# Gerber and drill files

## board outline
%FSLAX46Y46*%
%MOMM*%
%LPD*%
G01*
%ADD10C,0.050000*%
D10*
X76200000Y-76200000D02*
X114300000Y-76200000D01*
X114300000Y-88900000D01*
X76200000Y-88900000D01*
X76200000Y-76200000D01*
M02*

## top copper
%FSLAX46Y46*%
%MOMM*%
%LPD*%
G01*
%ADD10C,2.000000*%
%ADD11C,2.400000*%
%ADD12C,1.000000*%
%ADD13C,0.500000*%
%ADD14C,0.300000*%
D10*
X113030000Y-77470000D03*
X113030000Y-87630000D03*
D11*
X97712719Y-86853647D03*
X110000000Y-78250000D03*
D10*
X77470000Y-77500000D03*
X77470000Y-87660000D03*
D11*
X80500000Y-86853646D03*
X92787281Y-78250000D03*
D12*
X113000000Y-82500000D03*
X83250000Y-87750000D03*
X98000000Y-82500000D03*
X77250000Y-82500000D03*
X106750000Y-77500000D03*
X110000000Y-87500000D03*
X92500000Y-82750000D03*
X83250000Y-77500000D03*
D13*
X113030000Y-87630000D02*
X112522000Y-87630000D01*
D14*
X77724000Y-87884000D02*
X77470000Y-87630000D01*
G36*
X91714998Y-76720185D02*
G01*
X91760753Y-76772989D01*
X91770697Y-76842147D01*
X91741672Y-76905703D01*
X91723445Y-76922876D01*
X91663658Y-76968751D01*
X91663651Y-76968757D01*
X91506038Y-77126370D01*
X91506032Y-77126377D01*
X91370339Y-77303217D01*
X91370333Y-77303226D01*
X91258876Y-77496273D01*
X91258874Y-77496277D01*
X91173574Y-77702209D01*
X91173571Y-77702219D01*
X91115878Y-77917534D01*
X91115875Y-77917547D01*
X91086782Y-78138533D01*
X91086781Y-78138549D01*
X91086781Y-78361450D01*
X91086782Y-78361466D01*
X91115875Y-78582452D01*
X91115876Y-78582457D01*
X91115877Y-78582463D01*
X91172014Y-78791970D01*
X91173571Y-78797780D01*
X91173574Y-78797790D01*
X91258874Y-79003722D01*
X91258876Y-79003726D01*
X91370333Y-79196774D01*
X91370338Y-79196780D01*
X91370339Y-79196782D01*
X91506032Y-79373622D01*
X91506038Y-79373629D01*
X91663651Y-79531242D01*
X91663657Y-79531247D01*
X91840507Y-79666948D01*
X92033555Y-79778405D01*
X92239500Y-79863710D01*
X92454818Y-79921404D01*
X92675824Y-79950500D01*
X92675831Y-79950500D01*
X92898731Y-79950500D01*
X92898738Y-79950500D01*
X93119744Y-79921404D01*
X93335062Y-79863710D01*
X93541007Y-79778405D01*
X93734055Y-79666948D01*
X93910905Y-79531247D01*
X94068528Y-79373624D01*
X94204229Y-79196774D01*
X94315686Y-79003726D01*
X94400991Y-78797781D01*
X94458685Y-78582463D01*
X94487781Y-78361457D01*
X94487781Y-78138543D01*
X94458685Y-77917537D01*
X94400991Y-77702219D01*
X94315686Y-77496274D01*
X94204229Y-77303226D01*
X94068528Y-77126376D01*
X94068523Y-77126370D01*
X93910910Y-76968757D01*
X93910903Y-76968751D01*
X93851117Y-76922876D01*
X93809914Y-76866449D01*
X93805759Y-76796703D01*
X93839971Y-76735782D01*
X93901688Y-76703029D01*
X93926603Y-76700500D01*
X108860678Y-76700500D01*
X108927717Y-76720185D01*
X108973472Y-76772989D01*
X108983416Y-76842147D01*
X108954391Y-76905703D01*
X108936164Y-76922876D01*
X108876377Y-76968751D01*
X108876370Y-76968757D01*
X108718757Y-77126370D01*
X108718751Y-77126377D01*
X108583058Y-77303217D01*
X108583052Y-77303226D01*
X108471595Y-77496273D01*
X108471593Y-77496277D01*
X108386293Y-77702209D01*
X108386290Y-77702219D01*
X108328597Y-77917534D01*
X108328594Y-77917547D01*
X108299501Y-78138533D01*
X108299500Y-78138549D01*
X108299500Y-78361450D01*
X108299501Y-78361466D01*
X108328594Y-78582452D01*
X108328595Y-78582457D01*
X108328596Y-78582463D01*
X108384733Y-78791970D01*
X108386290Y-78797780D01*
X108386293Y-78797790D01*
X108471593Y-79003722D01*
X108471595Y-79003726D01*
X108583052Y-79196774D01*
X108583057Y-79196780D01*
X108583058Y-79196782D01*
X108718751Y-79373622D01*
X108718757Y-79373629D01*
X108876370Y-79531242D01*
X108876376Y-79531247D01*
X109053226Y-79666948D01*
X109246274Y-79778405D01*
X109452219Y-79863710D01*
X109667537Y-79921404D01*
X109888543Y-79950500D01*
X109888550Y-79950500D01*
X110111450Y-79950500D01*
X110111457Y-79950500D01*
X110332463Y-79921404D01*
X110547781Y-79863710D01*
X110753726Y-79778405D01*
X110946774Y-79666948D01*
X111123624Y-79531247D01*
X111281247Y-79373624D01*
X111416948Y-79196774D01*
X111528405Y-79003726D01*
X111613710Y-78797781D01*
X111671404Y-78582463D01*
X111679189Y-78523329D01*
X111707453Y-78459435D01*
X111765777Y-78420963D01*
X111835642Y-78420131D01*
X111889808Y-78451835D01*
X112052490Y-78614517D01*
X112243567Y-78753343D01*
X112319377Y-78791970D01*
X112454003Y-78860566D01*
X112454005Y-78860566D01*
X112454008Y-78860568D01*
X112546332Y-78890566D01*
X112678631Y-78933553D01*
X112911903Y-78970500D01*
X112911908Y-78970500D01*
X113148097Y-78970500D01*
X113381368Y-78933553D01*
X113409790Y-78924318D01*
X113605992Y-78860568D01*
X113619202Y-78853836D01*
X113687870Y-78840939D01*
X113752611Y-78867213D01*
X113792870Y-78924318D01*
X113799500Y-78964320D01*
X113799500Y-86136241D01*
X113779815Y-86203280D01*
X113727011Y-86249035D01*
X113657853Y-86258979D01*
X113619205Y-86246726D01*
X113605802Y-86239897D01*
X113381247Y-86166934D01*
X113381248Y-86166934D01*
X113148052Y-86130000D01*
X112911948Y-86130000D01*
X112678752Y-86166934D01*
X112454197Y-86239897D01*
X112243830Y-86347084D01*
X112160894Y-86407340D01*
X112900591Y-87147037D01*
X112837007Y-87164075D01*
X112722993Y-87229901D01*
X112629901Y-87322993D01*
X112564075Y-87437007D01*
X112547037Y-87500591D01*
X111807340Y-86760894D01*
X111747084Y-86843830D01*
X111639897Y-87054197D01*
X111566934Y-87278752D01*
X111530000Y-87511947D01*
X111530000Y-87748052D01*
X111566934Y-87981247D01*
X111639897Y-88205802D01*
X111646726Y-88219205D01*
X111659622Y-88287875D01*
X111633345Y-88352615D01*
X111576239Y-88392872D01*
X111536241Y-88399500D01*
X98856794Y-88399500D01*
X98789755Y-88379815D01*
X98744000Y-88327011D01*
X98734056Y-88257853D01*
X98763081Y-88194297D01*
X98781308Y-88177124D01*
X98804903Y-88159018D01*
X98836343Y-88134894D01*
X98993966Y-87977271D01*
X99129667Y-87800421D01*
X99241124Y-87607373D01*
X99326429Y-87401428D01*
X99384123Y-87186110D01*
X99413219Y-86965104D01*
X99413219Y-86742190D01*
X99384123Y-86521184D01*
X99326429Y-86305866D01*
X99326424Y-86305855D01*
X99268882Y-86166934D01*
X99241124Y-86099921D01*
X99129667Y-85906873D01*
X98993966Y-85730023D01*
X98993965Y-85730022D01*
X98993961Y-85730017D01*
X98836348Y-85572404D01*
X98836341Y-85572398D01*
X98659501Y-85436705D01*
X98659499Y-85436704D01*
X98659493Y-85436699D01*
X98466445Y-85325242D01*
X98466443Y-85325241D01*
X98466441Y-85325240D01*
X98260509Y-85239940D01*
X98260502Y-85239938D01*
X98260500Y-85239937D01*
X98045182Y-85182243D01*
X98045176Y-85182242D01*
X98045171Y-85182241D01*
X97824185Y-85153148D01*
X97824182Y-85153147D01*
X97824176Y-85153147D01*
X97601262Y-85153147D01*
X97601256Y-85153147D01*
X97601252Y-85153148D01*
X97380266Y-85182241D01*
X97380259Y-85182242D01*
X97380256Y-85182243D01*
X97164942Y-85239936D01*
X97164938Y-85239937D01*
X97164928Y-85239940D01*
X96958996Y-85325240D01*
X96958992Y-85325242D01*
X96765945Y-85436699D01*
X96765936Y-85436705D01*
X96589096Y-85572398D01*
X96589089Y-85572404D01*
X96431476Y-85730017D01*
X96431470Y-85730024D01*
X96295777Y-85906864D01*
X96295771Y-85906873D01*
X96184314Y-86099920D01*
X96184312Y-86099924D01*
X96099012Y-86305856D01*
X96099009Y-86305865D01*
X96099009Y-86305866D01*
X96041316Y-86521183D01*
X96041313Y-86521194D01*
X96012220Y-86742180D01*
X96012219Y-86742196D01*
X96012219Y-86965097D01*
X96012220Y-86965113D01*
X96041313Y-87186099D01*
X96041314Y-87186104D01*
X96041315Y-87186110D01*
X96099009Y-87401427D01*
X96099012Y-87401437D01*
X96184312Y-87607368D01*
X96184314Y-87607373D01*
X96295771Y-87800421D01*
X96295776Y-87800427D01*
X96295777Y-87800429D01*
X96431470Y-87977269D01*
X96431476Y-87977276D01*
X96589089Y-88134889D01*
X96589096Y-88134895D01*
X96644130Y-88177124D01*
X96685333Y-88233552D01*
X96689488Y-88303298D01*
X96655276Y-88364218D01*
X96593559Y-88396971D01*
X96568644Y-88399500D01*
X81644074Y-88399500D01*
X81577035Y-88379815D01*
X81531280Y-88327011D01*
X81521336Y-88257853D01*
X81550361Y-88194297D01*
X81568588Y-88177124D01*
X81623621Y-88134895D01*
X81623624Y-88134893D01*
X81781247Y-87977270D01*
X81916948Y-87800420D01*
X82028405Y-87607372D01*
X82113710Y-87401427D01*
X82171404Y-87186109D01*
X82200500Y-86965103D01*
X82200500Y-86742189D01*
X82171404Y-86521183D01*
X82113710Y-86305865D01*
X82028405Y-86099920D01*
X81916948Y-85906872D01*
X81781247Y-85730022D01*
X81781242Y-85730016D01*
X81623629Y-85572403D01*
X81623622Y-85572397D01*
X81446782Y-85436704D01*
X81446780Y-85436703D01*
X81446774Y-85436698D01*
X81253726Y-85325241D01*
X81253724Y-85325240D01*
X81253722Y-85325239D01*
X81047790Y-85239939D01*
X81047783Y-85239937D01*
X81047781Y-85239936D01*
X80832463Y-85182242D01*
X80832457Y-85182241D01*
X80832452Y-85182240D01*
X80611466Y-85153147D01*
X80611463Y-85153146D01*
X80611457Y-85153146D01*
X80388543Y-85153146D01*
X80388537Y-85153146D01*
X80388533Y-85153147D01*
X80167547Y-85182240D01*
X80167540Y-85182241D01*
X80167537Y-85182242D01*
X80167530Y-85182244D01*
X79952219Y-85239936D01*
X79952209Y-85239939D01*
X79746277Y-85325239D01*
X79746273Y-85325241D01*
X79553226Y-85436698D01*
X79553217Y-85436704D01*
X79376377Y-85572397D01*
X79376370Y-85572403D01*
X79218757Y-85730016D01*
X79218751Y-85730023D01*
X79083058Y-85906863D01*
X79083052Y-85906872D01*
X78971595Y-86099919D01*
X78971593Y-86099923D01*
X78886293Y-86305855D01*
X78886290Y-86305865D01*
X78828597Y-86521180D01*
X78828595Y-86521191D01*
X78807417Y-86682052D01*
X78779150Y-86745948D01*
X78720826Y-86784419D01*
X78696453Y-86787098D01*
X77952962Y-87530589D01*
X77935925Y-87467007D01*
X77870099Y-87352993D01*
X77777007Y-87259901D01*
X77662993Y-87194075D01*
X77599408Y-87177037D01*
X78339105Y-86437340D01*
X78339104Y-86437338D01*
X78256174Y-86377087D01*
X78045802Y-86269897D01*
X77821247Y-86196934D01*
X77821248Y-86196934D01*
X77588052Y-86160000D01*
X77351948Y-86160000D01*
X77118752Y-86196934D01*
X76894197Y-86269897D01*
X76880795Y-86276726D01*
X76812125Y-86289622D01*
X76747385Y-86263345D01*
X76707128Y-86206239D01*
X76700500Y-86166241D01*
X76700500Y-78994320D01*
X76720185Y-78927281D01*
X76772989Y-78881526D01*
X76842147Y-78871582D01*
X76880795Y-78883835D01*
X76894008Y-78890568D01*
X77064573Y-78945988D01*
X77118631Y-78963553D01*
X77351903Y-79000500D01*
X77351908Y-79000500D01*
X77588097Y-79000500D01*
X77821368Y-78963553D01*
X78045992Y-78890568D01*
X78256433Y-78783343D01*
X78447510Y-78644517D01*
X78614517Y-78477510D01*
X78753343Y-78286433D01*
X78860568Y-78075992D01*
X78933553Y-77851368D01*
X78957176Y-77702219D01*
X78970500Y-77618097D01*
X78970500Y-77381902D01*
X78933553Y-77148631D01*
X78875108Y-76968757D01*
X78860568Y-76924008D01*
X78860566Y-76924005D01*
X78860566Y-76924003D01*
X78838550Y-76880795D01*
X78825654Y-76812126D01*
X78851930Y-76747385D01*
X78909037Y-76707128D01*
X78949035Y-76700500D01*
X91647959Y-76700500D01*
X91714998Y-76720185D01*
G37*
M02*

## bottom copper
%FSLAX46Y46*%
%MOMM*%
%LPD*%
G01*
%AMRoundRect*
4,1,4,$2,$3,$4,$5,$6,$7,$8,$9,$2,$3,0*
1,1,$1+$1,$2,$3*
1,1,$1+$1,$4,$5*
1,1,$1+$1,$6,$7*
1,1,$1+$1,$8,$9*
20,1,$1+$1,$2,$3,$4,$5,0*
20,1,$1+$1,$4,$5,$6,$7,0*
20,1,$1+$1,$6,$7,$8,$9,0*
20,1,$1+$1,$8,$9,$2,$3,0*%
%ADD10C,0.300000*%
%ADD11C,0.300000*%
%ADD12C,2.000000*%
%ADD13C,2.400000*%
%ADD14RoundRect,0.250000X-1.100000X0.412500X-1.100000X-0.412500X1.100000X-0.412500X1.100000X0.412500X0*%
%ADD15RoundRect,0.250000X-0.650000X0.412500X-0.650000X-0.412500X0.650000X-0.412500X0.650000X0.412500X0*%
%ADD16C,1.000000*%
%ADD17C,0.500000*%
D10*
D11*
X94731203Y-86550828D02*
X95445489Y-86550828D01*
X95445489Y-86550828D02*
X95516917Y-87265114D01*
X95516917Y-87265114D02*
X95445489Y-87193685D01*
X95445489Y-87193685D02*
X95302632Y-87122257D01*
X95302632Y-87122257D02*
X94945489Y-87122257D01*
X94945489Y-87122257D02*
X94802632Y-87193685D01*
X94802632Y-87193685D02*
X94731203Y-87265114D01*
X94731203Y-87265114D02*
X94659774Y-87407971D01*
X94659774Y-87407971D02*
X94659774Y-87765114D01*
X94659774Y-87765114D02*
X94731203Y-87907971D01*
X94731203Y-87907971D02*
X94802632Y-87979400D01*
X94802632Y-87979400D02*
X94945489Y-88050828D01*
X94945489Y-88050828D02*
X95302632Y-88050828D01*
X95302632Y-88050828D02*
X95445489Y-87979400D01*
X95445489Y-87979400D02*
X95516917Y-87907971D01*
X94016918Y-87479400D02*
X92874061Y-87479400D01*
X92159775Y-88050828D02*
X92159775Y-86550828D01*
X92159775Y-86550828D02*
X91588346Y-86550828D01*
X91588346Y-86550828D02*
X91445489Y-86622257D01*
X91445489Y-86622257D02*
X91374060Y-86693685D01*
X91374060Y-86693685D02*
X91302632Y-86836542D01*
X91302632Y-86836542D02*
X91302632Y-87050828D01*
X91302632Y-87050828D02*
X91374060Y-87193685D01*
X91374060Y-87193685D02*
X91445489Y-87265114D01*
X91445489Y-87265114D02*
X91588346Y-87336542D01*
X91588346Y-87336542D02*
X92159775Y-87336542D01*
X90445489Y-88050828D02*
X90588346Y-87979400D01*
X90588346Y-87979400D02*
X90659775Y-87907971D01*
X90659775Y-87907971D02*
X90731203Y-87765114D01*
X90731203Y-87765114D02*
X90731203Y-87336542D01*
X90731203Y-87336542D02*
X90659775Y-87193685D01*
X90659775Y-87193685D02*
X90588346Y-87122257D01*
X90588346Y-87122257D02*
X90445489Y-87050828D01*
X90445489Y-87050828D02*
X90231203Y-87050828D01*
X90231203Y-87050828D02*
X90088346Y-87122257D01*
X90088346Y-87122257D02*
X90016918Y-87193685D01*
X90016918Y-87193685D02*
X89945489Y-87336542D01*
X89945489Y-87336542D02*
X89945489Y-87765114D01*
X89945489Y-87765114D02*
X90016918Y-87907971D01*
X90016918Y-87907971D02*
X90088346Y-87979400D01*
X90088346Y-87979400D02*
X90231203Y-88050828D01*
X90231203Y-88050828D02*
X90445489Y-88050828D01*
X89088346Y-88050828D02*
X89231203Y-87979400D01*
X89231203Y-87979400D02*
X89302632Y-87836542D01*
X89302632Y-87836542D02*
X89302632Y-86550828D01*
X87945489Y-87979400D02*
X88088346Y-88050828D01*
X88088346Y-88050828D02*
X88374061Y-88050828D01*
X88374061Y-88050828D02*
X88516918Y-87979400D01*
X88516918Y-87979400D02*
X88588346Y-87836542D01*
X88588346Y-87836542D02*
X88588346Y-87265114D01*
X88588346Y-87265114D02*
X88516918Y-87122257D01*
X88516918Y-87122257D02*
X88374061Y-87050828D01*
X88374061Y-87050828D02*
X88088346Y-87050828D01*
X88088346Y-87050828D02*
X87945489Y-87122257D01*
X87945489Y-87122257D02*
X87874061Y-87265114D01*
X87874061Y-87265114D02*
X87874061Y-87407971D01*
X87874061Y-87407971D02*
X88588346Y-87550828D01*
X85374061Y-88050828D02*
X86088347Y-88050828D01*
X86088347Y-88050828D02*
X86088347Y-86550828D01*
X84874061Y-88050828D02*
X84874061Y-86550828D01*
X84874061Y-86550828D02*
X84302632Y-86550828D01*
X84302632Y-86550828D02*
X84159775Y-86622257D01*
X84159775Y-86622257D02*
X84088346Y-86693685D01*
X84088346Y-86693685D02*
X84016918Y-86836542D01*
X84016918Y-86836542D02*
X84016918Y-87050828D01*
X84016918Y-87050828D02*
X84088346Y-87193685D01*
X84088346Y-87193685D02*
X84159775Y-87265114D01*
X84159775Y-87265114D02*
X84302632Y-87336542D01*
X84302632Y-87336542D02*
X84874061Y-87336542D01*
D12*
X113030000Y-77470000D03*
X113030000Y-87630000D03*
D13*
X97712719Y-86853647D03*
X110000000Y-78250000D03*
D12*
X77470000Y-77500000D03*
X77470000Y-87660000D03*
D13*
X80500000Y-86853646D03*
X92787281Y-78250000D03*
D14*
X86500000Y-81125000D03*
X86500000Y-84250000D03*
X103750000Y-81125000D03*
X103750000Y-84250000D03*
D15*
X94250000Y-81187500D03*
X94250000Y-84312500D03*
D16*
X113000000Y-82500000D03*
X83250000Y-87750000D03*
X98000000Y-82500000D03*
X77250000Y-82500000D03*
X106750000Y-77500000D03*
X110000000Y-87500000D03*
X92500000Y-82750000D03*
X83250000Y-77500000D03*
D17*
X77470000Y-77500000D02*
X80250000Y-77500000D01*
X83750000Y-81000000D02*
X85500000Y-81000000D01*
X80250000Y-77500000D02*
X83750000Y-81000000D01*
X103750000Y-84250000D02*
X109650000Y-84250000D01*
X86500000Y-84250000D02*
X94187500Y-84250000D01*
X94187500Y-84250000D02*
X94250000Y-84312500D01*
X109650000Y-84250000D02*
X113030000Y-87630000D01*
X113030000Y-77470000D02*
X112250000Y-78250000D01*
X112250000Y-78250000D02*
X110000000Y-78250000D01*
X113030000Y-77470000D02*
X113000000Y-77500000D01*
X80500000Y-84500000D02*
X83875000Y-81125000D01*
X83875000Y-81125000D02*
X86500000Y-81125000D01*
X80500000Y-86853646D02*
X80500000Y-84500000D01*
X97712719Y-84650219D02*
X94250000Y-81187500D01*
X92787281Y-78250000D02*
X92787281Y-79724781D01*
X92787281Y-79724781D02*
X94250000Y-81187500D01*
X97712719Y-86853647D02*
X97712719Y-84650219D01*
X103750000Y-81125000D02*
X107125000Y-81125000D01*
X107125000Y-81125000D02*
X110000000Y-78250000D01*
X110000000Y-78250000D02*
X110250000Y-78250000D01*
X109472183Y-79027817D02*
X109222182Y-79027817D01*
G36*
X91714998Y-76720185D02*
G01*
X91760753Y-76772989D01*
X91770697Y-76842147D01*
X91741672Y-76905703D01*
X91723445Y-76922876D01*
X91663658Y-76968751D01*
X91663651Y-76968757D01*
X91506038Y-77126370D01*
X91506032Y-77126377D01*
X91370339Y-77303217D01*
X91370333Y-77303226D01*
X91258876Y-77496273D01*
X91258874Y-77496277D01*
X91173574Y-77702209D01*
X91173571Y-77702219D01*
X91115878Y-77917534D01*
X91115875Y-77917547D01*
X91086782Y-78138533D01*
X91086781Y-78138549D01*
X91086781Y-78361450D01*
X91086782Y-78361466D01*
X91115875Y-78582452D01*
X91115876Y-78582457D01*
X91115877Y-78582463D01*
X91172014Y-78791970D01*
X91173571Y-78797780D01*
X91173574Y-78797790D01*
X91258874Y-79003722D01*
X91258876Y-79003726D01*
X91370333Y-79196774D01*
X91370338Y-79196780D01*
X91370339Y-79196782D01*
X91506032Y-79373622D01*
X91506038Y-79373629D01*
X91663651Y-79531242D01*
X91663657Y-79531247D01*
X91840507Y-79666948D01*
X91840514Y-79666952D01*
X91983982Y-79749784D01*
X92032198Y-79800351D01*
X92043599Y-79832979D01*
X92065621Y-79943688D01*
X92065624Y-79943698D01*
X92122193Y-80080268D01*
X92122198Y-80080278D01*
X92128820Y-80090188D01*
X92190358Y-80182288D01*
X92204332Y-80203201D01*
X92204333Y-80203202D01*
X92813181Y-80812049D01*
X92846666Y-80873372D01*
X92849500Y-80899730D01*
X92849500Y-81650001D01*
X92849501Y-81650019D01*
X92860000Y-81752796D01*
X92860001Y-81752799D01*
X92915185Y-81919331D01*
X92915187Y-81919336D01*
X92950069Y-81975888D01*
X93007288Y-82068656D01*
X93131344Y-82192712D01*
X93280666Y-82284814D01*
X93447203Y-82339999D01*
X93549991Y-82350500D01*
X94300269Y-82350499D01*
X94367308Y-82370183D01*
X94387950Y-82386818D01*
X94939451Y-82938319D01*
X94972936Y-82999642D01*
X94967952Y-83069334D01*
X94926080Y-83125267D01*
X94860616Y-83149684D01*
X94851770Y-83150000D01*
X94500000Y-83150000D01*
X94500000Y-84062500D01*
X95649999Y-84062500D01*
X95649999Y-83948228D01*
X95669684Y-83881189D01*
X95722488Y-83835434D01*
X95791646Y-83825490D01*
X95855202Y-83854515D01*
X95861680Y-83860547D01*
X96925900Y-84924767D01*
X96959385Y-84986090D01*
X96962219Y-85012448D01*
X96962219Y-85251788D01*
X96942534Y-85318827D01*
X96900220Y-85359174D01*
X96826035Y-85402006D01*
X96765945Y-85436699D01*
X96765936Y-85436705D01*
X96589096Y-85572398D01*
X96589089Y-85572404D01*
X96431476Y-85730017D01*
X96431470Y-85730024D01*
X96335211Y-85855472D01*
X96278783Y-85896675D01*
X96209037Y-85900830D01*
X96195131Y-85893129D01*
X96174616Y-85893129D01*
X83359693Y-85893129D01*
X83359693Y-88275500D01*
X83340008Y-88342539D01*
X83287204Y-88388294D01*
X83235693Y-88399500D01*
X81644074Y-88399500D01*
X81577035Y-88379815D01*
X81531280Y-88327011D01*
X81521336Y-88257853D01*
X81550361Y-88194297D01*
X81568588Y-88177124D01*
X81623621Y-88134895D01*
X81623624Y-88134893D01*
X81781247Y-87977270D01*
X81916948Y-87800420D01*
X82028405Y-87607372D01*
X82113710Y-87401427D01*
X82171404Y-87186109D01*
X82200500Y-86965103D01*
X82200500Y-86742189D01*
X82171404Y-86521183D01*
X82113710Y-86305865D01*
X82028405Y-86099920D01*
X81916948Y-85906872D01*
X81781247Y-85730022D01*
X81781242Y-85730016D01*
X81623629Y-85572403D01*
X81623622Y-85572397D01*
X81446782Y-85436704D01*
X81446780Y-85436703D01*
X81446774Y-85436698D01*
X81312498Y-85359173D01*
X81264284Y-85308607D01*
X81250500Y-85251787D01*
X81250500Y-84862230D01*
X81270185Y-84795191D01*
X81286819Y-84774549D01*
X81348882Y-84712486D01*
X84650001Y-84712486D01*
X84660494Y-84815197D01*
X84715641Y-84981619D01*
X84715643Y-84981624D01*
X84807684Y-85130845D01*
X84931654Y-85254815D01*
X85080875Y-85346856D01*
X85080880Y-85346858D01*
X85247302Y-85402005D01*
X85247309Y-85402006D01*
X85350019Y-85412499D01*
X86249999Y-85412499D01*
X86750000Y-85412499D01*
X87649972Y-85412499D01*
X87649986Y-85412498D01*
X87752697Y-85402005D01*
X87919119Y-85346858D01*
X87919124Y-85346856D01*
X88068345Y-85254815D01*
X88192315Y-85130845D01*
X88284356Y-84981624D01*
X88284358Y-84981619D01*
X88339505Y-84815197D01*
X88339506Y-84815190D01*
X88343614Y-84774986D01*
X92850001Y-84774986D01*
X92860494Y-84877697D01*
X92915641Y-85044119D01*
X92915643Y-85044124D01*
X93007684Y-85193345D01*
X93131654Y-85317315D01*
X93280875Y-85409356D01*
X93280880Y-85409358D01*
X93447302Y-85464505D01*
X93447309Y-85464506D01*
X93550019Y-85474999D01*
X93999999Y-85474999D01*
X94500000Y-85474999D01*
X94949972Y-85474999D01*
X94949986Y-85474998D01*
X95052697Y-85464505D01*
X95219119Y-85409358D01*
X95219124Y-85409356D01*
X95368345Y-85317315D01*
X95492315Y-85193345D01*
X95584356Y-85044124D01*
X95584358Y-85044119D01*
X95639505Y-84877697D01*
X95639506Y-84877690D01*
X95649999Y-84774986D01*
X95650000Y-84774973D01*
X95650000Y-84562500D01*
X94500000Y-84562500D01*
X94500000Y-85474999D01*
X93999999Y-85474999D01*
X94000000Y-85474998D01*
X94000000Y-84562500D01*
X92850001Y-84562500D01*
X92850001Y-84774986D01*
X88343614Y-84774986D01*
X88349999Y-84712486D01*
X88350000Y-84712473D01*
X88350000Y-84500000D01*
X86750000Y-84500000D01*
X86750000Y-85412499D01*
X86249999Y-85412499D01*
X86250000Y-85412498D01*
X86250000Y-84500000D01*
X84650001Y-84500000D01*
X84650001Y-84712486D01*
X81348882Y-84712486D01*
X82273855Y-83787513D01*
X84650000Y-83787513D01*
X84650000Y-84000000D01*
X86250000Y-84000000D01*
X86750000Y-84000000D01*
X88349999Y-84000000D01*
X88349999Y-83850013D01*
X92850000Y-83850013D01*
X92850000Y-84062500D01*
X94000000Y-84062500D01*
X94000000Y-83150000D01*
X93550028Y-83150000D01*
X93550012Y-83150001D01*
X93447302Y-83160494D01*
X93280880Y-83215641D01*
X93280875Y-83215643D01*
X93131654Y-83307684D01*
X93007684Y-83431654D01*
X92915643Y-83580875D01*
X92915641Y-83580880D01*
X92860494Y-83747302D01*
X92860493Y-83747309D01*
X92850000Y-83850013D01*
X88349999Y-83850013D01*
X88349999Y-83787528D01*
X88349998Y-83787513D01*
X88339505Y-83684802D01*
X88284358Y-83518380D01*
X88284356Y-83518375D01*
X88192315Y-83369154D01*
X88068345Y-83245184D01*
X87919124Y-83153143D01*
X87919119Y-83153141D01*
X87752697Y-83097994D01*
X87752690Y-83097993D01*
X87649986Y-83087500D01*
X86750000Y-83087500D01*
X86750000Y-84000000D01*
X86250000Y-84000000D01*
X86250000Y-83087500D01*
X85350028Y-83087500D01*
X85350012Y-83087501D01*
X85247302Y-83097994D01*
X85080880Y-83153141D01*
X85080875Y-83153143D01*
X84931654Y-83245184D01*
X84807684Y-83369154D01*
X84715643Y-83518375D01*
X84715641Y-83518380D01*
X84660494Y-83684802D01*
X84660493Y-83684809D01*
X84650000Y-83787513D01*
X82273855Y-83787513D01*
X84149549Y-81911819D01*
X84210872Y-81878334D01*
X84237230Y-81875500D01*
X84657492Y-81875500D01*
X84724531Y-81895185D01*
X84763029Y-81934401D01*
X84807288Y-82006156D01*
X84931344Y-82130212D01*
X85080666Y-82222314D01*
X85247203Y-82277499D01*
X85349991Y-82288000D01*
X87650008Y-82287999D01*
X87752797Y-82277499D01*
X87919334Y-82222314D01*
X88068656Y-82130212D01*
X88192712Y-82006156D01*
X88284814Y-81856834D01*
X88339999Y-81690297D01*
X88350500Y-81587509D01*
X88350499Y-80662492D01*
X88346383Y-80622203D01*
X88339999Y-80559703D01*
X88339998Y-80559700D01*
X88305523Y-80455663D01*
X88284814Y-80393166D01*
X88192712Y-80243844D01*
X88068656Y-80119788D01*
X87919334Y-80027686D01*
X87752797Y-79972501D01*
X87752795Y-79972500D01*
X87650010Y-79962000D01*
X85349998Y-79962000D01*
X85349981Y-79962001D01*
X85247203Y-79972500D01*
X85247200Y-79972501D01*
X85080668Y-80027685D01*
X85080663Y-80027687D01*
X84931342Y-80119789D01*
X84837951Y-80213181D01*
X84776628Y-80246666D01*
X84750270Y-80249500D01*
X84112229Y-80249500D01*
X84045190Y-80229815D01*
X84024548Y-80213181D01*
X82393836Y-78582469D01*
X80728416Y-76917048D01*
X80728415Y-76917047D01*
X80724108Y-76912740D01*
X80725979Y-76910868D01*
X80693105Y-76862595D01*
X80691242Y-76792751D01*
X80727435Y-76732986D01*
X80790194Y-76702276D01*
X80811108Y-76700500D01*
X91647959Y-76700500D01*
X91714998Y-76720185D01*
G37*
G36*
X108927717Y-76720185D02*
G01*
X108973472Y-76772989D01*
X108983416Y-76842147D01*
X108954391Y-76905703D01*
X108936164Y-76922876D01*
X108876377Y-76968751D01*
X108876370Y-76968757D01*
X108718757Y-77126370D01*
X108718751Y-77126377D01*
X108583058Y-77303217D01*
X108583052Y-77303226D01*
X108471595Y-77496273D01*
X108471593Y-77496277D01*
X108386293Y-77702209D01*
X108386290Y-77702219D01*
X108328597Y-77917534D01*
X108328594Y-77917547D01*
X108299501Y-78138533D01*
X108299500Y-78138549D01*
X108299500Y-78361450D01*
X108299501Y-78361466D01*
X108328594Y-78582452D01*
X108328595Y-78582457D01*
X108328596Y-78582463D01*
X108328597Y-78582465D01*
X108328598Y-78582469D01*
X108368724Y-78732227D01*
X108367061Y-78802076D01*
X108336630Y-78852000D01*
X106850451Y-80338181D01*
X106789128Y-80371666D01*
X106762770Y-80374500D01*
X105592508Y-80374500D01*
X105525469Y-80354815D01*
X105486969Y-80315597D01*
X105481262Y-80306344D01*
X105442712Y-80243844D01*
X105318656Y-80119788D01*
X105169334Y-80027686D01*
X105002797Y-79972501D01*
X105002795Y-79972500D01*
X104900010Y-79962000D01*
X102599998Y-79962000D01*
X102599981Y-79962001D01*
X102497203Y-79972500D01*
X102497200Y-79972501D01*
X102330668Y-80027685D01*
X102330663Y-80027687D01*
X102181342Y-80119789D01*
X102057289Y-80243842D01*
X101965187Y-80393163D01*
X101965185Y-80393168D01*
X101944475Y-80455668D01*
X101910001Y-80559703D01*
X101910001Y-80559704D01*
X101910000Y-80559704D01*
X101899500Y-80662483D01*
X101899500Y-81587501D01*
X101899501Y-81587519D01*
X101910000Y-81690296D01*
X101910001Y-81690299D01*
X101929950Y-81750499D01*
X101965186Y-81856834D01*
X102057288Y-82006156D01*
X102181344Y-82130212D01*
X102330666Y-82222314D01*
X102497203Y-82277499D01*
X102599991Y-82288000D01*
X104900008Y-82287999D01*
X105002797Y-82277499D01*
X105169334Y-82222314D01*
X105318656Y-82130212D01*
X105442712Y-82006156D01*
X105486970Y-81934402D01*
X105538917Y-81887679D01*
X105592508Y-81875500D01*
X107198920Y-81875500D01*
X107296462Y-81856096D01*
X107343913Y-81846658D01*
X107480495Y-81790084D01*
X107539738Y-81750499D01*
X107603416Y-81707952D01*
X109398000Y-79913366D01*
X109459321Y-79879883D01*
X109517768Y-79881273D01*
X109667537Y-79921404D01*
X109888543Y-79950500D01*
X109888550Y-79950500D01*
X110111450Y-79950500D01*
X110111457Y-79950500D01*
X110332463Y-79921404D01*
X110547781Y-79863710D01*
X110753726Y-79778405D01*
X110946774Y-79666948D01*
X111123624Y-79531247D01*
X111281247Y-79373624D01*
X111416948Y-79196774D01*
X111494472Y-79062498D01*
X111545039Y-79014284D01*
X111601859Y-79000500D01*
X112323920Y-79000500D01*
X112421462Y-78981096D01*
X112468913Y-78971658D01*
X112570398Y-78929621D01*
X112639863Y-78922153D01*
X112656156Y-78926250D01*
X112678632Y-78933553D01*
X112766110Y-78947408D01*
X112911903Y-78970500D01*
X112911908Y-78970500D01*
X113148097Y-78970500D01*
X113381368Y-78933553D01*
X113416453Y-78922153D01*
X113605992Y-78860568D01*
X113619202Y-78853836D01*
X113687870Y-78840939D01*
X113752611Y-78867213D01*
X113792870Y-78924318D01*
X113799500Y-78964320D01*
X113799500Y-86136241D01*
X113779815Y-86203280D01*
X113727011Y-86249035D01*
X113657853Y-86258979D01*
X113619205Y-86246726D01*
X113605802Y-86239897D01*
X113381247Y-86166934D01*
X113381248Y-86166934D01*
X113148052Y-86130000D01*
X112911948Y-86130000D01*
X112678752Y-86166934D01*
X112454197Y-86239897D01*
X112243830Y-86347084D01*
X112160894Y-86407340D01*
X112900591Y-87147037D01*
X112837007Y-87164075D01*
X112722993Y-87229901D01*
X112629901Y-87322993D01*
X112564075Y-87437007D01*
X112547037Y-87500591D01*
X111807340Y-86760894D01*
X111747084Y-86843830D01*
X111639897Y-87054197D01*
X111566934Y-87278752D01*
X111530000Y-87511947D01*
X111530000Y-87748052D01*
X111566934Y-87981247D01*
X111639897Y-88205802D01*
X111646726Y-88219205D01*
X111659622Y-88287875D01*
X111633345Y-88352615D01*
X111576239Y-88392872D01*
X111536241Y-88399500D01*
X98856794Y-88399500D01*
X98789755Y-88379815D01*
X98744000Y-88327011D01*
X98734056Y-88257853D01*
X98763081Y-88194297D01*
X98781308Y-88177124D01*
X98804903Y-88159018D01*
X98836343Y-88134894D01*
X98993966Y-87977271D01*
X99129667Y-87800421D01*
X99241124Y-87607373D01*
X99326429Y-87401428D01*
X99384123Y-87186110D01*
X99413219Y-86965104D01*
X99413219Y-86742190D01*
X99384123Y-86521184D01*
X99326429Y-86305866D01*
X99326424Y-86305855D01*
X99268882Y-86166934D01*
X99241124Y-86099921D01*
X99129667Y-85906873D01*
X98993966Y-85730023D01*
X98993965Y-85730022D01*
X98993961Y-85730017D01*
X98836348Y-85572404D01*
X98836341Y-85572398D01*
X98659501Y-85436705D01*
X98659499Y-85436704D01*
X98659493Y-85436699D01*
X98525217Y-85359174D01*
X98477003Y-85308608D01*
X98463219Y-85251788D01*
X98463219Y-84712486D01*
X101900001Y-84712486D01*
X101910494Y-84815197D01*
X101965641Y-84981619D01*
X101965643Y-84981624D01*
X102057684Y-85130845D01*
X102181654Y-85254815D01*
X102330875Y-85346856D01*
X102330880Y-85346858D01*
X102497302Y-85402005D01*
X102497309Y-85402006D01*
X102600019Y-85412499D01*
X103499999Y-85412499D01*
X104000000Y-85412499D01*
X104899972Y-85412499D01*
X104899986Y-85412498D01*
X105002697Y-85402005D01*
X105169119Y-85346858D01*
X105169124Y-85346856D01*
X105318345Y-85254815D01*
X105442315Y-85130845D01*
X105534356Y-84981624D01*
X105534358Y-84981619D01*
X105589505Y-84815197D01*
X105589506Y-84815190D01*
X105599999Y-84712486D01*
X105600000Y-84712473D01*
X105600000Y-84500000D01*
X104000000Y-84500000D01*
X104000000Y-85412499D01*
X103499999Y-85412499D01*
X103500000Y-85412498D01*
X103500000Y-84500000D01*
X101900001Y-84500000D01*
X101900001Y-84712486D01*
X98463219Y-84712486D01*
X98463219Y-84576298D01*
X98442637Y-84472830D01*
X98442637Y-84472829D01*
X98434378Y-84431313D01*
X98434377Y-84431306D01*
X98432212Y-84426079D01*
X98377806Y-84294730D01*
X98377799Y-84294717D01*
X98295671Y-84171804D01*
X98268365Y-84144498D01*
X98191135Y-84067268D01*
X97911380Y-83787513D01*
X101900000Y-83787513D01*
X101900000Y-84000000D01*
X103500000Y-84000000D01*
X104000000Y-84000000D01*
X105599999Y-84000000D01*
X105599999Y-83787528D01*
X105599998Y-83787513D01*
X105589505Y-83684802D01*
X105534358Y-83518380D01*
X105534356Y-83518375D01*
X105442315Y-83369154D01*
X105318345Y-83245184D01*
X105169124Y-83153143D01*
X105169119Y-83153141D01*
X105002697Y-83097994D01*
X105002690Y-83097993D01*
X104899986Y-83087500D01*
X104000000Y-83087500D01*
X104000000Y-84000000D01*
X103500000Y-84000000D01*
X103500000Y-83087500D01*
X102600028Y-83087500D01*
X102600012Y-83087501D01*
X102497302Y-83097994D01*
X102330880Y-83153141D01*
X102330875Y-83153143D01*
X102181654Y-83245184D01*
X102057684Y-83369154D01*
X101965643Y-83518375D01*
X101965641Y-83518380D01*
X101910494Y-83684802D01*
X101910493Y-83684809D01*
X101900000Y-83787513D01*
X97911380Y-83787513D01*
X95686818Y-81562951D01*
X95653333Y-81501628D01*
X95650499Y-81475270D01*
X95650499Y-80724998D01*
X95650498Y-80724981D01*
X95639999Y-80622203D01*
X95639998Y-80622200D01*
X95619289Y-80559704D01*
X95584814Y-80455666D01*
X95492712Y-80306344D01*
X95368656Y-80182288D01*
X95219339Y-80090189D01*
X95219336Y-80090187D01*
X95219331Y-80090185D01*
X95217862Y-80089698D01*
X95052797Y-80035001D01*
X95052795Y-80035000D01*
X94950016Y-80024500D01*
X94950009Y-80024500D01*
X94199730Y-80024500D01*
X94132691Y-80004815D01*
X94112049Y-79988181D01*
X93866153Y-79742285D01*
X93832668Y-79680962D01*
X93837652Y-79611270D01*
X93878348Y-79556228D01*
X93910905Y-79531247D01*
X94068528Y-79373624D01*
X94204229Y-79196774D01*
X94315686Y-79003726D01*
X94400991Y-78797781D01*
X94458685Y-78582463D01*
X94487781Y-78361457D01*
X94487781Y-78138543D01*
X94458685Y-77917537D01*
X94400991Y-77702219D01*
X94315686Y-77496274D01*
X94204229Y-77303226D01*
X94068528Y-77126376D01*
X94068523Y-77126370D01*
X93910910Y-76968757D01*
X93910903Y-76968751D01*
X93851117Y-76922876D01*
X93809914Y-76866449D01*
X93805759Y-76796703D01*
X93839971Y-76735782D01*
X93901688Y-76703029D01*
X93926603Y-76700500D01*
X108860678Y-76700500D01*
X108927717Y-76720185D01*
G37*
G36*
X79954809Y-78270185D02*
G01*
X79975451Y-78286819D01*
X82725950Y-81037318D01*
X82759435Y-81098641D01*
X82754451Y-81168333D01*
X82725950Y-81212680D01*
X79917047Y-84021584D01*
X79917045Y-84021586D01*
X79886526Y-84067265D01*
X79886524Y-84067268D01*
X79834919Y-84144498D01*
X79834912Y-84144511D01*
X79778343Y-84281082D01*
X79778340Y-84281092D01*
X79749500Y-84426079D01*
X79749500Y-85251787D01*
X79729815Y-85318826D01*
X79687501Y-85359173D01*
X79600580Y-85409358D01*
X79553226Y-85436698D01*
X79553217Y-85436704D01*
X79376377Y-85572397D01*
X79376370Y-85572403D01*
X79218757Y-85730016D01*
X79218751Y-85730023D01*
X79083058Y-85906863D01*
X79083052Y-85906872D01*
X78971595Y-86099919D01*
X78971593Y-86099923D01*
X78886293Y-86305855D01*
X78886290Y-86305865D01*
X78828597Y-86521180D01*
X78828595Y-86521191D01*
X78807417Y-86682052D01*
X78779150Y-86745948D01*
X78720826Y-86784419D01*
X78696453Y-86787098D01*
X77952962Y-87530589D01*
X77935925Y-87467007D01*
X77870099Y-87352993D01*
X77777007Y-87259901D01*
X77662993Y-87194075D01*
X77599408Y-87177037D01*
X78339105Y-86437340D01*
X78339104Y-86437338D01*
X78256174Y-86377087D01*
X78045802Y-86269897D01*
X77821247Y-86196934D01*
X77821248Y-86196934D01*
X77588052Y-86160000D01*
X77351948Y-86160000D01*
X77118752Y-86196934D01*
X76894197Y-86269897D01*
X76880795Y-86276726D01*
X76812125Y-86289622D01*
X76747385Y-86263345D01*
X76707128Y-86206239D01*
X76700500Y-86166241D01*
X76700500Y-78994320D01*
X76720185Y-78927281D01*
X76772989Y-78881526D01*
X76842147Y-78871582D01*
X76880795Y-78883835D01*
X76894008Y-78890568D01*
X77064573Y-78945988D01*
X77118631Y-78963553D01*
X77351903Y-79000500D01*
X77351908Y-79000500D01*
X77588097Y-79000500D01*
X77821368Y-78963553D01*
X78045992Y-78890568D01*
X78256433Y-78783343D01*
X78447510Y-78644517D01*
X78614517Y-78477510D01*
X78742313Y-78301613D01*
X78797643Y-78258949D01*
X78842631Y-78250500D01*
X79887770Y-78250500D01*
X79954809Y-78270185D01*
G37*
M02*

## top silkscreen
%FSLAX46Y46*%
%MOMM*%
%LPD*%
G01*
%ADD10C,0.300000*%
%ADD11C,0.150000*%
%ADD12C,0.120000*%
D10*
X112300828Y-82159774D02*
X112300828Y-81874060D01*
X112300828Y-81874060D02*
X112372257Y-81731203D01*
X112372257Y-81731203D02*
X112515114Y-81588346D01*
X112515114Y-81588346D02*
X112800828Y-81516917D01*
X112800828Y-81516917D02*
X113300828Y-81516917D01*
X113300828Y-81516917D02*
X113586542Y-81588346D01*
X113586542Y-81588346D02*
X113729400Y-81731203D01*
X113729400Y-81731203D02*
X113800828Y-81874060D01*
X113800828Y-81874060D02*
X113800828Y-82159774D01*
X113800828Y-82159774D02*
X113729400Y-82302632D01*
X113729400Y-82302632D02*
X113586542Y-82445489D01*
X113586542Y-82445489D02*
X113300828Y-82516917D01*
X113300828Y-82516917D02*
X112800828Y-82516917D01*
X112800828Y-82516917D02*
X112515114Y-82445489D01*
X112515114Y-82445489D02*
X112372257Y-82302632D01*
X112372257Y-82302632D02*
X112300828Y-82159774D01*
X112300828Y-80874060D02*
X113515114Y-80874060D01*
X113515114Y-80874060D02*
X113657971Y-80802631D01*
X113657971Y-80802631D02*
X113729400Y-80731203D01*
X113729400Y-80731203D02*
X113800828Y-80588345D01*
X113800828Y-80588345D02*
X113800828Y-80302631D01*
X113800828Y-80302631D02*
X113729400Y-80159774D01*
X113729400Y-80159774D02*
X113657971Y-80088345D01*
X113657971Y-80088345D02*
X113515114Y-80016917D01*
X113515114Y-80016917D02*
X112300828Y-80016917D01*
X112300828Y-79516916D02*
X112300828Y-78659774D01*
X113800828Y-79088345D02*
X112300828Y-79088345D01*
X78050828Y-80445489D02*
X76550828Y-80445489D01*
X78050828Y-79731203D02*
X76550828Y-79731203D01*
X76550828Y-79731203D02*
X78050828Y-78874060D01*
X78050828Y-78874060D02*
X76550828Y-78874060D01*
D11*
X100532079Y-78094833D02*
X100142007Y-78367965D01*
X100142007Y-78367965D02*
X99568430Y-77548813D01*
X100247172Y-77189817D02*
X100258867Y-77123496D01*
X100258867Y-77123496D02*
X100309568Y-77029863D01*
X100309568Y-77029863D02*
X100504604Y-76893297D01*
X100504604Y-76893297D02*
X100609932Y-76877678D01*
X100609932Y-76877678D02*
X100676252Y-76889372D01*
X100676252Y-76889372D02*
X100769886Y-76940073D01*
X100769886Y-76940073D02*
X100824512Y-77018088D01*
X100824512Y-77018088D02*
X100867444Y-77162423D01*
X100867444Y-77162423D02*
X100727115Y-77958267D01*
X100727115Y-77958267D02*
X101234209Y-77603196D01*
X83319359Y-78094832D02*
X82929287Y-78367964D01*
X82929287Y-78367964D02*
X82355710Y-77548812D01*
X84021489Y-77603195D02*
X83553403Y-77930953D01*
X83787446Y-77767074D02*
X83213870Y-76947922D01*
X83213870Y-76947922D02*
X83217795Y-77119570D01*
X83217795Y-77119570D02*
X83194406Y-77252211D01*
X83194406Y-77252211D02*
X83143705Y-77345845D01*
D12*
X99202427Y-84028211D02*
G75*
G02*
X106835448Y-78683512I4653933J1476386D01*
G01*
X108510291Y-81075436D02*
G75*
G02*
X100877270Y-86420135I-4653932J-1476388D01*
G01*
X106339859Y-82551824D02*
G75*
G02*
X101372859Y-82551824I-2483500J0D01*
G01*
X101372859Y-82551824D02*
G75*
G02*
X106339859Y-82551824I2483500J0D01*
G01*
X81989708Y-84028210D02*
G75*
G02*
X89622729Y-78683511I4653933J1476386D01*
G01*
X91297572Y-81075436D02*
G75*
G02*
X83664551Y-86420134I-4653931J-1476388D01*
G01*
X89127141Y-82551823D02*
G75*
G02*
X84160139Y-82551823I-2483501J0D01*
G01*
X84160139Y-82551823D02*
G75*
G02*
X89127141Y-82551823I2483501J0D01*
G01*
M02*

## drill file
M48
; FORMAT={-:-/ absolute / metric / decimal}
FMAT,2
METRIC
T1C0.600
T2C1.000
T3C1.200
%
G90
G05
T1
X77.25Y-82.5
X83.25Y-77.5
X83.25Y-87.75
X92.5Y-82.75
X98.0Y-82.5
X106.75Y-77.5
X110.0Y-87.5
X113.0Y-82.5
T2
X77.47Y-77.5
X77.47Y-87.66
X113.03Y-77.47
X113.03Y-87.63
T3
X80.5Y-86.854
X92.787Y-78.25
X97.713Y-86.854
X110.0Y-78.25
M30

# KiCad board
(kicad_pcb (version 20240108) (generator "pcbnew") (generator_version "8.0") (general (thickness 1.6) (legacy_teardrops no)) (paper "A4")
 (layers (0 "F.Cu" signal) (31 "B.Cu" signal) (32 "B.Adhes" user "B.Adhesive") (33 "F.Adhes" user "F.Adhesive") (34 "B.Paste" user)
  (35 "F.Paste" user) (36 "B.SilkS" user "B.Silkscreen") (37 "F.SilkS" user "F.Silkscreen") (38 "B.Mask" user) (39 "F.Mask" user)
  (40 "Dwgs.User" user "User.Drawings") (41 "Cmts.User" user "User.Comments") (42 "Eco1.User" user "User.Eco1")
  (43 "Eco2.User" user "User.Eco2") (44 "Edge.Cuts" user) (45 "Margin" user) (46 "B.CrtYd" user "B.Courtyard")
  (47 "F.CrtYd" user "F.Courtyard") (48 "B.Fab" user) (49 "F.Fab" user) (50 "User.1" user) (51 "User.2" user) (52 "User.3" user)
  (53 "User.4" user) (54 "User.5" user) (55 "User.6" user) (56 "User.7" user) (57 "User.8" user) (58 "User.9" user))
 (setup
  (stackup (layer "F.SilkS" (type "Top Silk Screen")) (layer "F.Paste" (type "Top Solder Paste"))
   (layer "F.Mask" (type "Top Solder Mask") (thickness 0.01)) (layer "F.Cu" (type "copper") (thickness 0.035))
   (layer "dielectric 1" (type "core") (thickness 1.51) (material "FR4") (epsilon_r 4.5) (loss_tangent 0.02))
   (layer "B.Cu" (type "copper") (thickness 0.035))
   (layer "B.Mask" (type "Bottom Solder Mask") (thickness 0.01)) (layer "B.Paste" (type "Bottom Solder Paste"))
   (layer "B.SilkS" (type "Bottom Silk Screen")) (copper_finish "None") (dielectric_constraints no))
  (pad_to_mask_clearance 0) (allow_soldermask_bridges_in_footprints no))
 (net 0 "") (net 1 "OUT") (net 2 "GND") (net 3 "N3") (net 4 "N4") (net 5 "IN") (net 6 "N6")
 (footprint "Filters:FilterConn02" (layer "F.Cu") (at 113.03 82.55)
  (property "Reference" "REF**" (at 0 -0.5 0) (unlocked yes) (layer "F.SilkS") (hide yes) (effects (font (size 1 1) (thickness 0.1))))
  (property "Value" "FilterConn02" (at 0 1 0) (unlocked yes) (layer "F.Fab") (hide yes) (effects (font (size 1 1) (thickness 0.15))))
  (pad "3" thru_hole circle (at 0 -5.08) (size 2 2) (drill 1) (layers "*.Cu" "*.Mask") (remove_unused_layers no) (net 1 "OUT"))
  (pad "4" thru_hole circle (at 0 5.08) (size 2 2) (drill 1) (layers "*.Cu" "*.Mask") (remove_unused_layers no) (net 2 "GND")))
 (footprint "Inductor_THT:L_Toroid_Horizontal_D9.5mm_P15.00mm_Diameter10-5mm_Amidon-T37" (layer "F.Cu") (at 97.712719 86.853647 35)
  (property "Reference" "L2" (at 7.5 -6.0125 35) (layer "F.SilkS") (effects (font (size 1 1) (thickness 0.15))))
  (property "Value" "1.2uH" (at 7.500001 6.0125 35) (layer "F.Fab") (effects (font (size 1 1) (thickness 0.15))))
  (fp_arc (start 2.840901 -1.46) (mid 7.5 -4.882499) (end 12.159099 -1.46) (stroke (width 0.12) (type solid)) (layer "F.SilkS"))
  (fp_arc (start 12.159099 1.46) (mid 7.5 4.8825) (end 2.840901 1.46) (stroke (width 0.12) (type solid)) (layer "F.SilkS"))
  (fp_circle (center 7.5 0) (end 9.983499 0) (stroke (width 0.12) (type solid)) (fill none) (layer "F.SilkS"))
  (pad "1" thru_hole circle (at 0 0 35) (size 2.4 2.4) (drill 1.2) (layers "*.Cu" "*.Mask") (remove_unused_layers no) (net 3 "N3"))
  (pad "2" thru_hole circle (at 15.000001 0 35) (size 2.4 2.4) (drill 1.2) (layers "*.Cu" "*.Mask") (remove_unused_layers no) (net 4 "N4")))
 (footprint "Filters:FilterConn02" (layer "F.Cu") (at 77.47 82.58)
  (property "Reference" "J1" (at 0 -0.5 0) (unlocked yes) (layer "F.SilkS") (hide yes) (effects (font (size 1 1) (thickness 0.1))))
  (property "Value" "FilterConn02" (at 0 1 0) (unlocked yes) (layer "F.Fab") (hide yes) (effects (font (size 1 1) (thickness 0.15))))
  (pad "1" thru_hole circle (at 0 -5.08) (size 2 2) (drill 1) (layers "*.Cu" "*.Mask") (remove_unused_layers no) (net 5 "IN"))
  (pad "2" thru_hole circle (at 0 5.08) (size 2 2) (drill 1) (layers "*.Cu" "*.Mask") (remove_unused_layers no) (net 2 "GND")))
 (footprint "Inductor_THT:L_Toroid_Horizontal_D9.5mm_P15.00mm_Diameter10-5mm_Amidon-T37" (layer "F.Cu") (at 80.5 86.853646 35)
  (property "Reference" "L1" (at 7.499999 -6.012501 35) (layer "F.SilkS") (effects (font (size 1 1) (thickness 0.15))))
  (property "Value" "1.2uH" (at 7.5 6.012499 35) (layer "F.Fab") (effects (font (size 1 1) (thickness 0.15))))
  (fp_arc (start 2.840901 -1.46) (mid 7.5 -4.882499) (end 12.159099 -1.46) (stroke (width 0.12) (type solid)) (layer "F.SilkS"))
  (fp_arc (start 12.159098 1.46) (mid 7.5 4.8825) (end 2.840901 1.46) (stroke (width 0.12) (type solid)) (layer "F.SilkS"))
  (fp_circle (center 7.5 0) (end 9.983501 0) (stroke (width 0.12) (type solid)) (fill none) (layer "F.SilkS"))
  (pad "1" thru_hole circle (at 0 0 35) (size 2.4 2.4) (drill 1.2) (layers "*.Cu" "*.Mask") (remove_unused_layers no) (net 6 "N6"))
  (pad "2" thru_hole circle (at 15 0.000001 35) (size 2.4 2.4) (drill 1.2) (layers "*.Cu" "*.Mask") (remove_unused_layers no) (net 3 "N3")))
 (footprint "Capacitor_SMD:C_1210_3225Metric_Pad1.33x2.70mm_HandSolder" (layer "B.Cu") (at 86.5 82.6875 -90)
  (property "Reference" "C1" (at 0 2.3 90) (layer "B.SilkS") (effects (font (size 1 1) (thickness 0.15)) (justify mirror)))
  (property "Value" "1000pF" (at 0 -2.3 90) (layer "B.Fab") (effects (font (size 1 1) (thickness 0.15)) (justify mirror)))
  (pad "1" smd roundrect (at -1.5625 0 270) (size 1.325 2.7) (layers "B.Cu" "B.Paste" "B.Mask") (roundrect_rratio 0.188679) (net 6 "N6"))
  (pad "2" smd roundrect (at 1.5625 0 270) (size 1.325 2.7) (layers "B.Cu" "B.Paste" "B.Mask") (roundrect_rratio 0.188679) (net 2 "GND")))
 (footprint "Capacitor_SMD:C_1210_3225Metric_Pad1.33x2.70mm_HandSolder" (layer "B.Cu") (at 103.75 82.6875 -90)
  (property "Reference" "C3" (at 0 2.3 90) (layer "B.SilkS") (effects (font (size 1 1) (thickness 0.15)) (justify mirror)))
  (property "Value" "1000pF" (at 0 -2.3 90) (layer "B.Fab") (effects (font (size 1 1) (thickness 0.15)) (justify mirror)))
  (pad "1" smd roundrect (at -1.5625 0 270) (size 1.325 2.7) (layers "B.Cu" "B.Paste" "B.Mask") (roundrect_rratio 0.188679) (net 4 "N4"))
  (pad "2" smd roundrect (at 1.5625 0 270) (size 1.325 2.7) (layers "B.Cu" "B.Paste" "B.Mask") (roundrect_rratio 0.188679) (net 2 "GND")))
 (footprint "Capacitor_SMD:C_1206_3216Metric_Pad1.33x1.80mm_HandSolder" (layer "B.Cu") (at 94.25 82.75 -90)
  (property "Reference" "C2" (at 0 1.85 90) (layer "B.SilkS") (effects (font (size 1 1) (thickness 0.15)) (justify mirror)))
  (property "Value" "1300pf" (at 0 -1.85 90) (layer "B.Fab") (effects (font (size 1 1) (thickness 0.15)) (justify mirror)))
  (pad "1" smd roundrect (at -1.5625 0 270) (size 1.325 1.8) (layers "B.Cu" "B.Paste" "B.Mask") (roundrect_rratio 0.188679) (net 3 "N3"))
  (pad "2" smd roundrect (at 1.5625 0 270) (size 1.325 1.8) (layers "B.Cu" "B.Paste" "B.Mask") (roundrect_rratio 0.188679) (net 2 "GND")))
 (gr_rect (start 76.2 76.2) (end 114.3 88.9) (stroke (width 0.05) (type default)) (fill none) (layer "Edge.Cuts"))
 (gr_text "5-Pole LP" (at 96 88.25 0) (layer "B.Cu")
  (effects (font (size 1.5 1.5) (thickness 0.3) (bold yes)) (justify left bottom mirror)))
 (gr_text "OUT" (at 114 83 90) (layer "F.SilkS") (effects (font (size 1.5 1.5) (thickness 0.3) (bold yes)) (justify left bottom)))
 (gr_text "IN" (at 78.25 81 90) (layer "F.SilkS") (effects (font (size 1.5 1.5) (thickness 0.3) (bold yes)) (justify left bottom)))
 (segment (start 77.47 77.5) (end 80.25 77.5) (width 0.5) (layer "B.Cu") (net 5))
 (segment (start 83.75 81) (end 85.5 81) (width 0.5) (layer "B.Cu") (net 5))
 (segment (start 80.25 77.5) (end 83.75 81) (width 0.5) (layer "B.Cu") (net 5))
 (segment (start 113.03 87.63) (end 112.522 87.63) (width 0.5) (layer "F.Cu") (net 2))
 (segment (start 77.724 87.884) (end 77.47 87.63) (width 0.3) (layer "F.Cu") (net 2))
 (via (at 113 82.5) (size 1) (drill 0.6) (layers "F.Cu" "B.Cu") (free yes) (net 2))
 (via (at 83.25 87.75) (size 1) (drill 0.6) (layers "F.Cu" "B.Cu") (free yes) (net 2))
 (via (at 98 82.5) (size 1) (drill 0.6) (layers "F.Cu" "B.Cu") (free yes) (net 2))
 (via (at 77.25 82.5) (size 1) (drill 0.6) (layers "F.Cu" "B.Cu") (free yes) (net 2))
 (via (at 106.75 77.5) (size 1) (drill 0.6) (layers "F.Cu" "B.Cu") (free yes) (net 2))
 (via (at 110 87.5) (size 1) (drill 0.6) (layers "F.Cu" "B.Cu") (free yes) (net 2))
 (via (at 92.5 82.75) (size 1) (drill 0.6) (layers "F.Cu" "B.Cu") (free yes) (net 2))
 (via (at 83.25 77.5) (size 1) (drill 0.6) (layers "F.Cu" "B.Cu") (free yes) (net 2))
 (segment (start 103.75 84.25) (end 109.65 84.25) (width 0.5) (layer "B.Cu") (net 2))
 (segment (start 86.5 84.25) (end 94.1875 84.25) (width 0.5) (layer "B.Cu") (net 2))
 (segment (start 94.1875 84.25) (end 94.25 84.3125) (width 0.5) (layer "B.Cu") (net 2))
 (segment (start 109.65 84.25) (end 113.03 87.63) (width 0.5) (layer "B.Cu") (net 2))
 (segment (start 113.03 77.47) (end 112.25 78.25) (width 0.5) (layer "B.Cu") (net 1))
 (segment (start 112.25 78.25) (end 110 78.25) (width 0.5) (layer "B.Cu") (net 1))
 (segment (start 113.03 77.47) (end 113 77.5) (width 0.5) (layer "B.Cu") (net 1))
 (segment (start 80.5 84.5) (end 83.875 81.125) (width 0.5) (layer "B.Cu") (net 6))
 (segment (start 83.875 81.125) (end 86.5 81.125) (width 0.5) (layer "B.Cu") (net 6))
 (segment (start 80.5 86.853646) (end 80.5 84.5) (width 0.5) (layer "B.Cu") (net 6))
 (segment (start 97.712719 84.650219) (end 94.25 81.1875) (width 0.5) (layer "B.Cu") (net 3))
 (segment (start 92.787281 78.25) (end 92.787281 79.724781) (width 0.5) (layer "B.Cu") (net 3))
 (segment (start 92.787281 79.724781) (end 94.25 81.1875) (width 0.5) (layer "B.Cu") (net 3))
 (segment (start 97.712719 86.853647) (end 97.712719 84.650219) (width 0.5) (layer "B.Cu") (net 3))
 (segment (start 103.75 81.125) (end 107.125 81.125) (width 0.5) (layer "B.Cu") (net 4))
 (segment (start 107.125 81.125) (end 110 78.25) (width 0.5) (layer "B.Cu") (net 4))
 (segment (start 110 78.25) (end 110.25 78.25) (width 0.5) (layer "B.Cu") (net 4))
 (segment (start 109.472183 79.027817) (end 109.222182 79.027817) (width 0.5) (layer "B.Cu") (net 4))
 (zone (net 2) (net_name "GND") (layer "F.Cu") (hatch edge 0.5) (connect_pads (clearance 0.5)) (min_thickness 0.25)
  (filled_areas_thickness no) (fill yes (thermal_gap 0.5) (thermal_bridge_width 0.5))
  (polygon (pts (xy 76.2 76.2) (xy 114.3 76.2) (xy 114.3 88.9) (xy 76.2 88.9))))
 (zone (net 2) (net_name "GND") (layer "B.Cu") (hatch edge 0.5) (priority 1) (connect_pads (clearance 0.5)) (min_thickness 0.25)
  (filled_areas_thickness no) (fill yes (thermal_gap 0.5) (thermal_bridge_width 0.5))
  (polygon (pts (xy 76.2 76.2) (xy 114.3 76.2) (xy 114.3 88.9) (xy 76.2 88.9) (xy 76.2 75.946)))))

